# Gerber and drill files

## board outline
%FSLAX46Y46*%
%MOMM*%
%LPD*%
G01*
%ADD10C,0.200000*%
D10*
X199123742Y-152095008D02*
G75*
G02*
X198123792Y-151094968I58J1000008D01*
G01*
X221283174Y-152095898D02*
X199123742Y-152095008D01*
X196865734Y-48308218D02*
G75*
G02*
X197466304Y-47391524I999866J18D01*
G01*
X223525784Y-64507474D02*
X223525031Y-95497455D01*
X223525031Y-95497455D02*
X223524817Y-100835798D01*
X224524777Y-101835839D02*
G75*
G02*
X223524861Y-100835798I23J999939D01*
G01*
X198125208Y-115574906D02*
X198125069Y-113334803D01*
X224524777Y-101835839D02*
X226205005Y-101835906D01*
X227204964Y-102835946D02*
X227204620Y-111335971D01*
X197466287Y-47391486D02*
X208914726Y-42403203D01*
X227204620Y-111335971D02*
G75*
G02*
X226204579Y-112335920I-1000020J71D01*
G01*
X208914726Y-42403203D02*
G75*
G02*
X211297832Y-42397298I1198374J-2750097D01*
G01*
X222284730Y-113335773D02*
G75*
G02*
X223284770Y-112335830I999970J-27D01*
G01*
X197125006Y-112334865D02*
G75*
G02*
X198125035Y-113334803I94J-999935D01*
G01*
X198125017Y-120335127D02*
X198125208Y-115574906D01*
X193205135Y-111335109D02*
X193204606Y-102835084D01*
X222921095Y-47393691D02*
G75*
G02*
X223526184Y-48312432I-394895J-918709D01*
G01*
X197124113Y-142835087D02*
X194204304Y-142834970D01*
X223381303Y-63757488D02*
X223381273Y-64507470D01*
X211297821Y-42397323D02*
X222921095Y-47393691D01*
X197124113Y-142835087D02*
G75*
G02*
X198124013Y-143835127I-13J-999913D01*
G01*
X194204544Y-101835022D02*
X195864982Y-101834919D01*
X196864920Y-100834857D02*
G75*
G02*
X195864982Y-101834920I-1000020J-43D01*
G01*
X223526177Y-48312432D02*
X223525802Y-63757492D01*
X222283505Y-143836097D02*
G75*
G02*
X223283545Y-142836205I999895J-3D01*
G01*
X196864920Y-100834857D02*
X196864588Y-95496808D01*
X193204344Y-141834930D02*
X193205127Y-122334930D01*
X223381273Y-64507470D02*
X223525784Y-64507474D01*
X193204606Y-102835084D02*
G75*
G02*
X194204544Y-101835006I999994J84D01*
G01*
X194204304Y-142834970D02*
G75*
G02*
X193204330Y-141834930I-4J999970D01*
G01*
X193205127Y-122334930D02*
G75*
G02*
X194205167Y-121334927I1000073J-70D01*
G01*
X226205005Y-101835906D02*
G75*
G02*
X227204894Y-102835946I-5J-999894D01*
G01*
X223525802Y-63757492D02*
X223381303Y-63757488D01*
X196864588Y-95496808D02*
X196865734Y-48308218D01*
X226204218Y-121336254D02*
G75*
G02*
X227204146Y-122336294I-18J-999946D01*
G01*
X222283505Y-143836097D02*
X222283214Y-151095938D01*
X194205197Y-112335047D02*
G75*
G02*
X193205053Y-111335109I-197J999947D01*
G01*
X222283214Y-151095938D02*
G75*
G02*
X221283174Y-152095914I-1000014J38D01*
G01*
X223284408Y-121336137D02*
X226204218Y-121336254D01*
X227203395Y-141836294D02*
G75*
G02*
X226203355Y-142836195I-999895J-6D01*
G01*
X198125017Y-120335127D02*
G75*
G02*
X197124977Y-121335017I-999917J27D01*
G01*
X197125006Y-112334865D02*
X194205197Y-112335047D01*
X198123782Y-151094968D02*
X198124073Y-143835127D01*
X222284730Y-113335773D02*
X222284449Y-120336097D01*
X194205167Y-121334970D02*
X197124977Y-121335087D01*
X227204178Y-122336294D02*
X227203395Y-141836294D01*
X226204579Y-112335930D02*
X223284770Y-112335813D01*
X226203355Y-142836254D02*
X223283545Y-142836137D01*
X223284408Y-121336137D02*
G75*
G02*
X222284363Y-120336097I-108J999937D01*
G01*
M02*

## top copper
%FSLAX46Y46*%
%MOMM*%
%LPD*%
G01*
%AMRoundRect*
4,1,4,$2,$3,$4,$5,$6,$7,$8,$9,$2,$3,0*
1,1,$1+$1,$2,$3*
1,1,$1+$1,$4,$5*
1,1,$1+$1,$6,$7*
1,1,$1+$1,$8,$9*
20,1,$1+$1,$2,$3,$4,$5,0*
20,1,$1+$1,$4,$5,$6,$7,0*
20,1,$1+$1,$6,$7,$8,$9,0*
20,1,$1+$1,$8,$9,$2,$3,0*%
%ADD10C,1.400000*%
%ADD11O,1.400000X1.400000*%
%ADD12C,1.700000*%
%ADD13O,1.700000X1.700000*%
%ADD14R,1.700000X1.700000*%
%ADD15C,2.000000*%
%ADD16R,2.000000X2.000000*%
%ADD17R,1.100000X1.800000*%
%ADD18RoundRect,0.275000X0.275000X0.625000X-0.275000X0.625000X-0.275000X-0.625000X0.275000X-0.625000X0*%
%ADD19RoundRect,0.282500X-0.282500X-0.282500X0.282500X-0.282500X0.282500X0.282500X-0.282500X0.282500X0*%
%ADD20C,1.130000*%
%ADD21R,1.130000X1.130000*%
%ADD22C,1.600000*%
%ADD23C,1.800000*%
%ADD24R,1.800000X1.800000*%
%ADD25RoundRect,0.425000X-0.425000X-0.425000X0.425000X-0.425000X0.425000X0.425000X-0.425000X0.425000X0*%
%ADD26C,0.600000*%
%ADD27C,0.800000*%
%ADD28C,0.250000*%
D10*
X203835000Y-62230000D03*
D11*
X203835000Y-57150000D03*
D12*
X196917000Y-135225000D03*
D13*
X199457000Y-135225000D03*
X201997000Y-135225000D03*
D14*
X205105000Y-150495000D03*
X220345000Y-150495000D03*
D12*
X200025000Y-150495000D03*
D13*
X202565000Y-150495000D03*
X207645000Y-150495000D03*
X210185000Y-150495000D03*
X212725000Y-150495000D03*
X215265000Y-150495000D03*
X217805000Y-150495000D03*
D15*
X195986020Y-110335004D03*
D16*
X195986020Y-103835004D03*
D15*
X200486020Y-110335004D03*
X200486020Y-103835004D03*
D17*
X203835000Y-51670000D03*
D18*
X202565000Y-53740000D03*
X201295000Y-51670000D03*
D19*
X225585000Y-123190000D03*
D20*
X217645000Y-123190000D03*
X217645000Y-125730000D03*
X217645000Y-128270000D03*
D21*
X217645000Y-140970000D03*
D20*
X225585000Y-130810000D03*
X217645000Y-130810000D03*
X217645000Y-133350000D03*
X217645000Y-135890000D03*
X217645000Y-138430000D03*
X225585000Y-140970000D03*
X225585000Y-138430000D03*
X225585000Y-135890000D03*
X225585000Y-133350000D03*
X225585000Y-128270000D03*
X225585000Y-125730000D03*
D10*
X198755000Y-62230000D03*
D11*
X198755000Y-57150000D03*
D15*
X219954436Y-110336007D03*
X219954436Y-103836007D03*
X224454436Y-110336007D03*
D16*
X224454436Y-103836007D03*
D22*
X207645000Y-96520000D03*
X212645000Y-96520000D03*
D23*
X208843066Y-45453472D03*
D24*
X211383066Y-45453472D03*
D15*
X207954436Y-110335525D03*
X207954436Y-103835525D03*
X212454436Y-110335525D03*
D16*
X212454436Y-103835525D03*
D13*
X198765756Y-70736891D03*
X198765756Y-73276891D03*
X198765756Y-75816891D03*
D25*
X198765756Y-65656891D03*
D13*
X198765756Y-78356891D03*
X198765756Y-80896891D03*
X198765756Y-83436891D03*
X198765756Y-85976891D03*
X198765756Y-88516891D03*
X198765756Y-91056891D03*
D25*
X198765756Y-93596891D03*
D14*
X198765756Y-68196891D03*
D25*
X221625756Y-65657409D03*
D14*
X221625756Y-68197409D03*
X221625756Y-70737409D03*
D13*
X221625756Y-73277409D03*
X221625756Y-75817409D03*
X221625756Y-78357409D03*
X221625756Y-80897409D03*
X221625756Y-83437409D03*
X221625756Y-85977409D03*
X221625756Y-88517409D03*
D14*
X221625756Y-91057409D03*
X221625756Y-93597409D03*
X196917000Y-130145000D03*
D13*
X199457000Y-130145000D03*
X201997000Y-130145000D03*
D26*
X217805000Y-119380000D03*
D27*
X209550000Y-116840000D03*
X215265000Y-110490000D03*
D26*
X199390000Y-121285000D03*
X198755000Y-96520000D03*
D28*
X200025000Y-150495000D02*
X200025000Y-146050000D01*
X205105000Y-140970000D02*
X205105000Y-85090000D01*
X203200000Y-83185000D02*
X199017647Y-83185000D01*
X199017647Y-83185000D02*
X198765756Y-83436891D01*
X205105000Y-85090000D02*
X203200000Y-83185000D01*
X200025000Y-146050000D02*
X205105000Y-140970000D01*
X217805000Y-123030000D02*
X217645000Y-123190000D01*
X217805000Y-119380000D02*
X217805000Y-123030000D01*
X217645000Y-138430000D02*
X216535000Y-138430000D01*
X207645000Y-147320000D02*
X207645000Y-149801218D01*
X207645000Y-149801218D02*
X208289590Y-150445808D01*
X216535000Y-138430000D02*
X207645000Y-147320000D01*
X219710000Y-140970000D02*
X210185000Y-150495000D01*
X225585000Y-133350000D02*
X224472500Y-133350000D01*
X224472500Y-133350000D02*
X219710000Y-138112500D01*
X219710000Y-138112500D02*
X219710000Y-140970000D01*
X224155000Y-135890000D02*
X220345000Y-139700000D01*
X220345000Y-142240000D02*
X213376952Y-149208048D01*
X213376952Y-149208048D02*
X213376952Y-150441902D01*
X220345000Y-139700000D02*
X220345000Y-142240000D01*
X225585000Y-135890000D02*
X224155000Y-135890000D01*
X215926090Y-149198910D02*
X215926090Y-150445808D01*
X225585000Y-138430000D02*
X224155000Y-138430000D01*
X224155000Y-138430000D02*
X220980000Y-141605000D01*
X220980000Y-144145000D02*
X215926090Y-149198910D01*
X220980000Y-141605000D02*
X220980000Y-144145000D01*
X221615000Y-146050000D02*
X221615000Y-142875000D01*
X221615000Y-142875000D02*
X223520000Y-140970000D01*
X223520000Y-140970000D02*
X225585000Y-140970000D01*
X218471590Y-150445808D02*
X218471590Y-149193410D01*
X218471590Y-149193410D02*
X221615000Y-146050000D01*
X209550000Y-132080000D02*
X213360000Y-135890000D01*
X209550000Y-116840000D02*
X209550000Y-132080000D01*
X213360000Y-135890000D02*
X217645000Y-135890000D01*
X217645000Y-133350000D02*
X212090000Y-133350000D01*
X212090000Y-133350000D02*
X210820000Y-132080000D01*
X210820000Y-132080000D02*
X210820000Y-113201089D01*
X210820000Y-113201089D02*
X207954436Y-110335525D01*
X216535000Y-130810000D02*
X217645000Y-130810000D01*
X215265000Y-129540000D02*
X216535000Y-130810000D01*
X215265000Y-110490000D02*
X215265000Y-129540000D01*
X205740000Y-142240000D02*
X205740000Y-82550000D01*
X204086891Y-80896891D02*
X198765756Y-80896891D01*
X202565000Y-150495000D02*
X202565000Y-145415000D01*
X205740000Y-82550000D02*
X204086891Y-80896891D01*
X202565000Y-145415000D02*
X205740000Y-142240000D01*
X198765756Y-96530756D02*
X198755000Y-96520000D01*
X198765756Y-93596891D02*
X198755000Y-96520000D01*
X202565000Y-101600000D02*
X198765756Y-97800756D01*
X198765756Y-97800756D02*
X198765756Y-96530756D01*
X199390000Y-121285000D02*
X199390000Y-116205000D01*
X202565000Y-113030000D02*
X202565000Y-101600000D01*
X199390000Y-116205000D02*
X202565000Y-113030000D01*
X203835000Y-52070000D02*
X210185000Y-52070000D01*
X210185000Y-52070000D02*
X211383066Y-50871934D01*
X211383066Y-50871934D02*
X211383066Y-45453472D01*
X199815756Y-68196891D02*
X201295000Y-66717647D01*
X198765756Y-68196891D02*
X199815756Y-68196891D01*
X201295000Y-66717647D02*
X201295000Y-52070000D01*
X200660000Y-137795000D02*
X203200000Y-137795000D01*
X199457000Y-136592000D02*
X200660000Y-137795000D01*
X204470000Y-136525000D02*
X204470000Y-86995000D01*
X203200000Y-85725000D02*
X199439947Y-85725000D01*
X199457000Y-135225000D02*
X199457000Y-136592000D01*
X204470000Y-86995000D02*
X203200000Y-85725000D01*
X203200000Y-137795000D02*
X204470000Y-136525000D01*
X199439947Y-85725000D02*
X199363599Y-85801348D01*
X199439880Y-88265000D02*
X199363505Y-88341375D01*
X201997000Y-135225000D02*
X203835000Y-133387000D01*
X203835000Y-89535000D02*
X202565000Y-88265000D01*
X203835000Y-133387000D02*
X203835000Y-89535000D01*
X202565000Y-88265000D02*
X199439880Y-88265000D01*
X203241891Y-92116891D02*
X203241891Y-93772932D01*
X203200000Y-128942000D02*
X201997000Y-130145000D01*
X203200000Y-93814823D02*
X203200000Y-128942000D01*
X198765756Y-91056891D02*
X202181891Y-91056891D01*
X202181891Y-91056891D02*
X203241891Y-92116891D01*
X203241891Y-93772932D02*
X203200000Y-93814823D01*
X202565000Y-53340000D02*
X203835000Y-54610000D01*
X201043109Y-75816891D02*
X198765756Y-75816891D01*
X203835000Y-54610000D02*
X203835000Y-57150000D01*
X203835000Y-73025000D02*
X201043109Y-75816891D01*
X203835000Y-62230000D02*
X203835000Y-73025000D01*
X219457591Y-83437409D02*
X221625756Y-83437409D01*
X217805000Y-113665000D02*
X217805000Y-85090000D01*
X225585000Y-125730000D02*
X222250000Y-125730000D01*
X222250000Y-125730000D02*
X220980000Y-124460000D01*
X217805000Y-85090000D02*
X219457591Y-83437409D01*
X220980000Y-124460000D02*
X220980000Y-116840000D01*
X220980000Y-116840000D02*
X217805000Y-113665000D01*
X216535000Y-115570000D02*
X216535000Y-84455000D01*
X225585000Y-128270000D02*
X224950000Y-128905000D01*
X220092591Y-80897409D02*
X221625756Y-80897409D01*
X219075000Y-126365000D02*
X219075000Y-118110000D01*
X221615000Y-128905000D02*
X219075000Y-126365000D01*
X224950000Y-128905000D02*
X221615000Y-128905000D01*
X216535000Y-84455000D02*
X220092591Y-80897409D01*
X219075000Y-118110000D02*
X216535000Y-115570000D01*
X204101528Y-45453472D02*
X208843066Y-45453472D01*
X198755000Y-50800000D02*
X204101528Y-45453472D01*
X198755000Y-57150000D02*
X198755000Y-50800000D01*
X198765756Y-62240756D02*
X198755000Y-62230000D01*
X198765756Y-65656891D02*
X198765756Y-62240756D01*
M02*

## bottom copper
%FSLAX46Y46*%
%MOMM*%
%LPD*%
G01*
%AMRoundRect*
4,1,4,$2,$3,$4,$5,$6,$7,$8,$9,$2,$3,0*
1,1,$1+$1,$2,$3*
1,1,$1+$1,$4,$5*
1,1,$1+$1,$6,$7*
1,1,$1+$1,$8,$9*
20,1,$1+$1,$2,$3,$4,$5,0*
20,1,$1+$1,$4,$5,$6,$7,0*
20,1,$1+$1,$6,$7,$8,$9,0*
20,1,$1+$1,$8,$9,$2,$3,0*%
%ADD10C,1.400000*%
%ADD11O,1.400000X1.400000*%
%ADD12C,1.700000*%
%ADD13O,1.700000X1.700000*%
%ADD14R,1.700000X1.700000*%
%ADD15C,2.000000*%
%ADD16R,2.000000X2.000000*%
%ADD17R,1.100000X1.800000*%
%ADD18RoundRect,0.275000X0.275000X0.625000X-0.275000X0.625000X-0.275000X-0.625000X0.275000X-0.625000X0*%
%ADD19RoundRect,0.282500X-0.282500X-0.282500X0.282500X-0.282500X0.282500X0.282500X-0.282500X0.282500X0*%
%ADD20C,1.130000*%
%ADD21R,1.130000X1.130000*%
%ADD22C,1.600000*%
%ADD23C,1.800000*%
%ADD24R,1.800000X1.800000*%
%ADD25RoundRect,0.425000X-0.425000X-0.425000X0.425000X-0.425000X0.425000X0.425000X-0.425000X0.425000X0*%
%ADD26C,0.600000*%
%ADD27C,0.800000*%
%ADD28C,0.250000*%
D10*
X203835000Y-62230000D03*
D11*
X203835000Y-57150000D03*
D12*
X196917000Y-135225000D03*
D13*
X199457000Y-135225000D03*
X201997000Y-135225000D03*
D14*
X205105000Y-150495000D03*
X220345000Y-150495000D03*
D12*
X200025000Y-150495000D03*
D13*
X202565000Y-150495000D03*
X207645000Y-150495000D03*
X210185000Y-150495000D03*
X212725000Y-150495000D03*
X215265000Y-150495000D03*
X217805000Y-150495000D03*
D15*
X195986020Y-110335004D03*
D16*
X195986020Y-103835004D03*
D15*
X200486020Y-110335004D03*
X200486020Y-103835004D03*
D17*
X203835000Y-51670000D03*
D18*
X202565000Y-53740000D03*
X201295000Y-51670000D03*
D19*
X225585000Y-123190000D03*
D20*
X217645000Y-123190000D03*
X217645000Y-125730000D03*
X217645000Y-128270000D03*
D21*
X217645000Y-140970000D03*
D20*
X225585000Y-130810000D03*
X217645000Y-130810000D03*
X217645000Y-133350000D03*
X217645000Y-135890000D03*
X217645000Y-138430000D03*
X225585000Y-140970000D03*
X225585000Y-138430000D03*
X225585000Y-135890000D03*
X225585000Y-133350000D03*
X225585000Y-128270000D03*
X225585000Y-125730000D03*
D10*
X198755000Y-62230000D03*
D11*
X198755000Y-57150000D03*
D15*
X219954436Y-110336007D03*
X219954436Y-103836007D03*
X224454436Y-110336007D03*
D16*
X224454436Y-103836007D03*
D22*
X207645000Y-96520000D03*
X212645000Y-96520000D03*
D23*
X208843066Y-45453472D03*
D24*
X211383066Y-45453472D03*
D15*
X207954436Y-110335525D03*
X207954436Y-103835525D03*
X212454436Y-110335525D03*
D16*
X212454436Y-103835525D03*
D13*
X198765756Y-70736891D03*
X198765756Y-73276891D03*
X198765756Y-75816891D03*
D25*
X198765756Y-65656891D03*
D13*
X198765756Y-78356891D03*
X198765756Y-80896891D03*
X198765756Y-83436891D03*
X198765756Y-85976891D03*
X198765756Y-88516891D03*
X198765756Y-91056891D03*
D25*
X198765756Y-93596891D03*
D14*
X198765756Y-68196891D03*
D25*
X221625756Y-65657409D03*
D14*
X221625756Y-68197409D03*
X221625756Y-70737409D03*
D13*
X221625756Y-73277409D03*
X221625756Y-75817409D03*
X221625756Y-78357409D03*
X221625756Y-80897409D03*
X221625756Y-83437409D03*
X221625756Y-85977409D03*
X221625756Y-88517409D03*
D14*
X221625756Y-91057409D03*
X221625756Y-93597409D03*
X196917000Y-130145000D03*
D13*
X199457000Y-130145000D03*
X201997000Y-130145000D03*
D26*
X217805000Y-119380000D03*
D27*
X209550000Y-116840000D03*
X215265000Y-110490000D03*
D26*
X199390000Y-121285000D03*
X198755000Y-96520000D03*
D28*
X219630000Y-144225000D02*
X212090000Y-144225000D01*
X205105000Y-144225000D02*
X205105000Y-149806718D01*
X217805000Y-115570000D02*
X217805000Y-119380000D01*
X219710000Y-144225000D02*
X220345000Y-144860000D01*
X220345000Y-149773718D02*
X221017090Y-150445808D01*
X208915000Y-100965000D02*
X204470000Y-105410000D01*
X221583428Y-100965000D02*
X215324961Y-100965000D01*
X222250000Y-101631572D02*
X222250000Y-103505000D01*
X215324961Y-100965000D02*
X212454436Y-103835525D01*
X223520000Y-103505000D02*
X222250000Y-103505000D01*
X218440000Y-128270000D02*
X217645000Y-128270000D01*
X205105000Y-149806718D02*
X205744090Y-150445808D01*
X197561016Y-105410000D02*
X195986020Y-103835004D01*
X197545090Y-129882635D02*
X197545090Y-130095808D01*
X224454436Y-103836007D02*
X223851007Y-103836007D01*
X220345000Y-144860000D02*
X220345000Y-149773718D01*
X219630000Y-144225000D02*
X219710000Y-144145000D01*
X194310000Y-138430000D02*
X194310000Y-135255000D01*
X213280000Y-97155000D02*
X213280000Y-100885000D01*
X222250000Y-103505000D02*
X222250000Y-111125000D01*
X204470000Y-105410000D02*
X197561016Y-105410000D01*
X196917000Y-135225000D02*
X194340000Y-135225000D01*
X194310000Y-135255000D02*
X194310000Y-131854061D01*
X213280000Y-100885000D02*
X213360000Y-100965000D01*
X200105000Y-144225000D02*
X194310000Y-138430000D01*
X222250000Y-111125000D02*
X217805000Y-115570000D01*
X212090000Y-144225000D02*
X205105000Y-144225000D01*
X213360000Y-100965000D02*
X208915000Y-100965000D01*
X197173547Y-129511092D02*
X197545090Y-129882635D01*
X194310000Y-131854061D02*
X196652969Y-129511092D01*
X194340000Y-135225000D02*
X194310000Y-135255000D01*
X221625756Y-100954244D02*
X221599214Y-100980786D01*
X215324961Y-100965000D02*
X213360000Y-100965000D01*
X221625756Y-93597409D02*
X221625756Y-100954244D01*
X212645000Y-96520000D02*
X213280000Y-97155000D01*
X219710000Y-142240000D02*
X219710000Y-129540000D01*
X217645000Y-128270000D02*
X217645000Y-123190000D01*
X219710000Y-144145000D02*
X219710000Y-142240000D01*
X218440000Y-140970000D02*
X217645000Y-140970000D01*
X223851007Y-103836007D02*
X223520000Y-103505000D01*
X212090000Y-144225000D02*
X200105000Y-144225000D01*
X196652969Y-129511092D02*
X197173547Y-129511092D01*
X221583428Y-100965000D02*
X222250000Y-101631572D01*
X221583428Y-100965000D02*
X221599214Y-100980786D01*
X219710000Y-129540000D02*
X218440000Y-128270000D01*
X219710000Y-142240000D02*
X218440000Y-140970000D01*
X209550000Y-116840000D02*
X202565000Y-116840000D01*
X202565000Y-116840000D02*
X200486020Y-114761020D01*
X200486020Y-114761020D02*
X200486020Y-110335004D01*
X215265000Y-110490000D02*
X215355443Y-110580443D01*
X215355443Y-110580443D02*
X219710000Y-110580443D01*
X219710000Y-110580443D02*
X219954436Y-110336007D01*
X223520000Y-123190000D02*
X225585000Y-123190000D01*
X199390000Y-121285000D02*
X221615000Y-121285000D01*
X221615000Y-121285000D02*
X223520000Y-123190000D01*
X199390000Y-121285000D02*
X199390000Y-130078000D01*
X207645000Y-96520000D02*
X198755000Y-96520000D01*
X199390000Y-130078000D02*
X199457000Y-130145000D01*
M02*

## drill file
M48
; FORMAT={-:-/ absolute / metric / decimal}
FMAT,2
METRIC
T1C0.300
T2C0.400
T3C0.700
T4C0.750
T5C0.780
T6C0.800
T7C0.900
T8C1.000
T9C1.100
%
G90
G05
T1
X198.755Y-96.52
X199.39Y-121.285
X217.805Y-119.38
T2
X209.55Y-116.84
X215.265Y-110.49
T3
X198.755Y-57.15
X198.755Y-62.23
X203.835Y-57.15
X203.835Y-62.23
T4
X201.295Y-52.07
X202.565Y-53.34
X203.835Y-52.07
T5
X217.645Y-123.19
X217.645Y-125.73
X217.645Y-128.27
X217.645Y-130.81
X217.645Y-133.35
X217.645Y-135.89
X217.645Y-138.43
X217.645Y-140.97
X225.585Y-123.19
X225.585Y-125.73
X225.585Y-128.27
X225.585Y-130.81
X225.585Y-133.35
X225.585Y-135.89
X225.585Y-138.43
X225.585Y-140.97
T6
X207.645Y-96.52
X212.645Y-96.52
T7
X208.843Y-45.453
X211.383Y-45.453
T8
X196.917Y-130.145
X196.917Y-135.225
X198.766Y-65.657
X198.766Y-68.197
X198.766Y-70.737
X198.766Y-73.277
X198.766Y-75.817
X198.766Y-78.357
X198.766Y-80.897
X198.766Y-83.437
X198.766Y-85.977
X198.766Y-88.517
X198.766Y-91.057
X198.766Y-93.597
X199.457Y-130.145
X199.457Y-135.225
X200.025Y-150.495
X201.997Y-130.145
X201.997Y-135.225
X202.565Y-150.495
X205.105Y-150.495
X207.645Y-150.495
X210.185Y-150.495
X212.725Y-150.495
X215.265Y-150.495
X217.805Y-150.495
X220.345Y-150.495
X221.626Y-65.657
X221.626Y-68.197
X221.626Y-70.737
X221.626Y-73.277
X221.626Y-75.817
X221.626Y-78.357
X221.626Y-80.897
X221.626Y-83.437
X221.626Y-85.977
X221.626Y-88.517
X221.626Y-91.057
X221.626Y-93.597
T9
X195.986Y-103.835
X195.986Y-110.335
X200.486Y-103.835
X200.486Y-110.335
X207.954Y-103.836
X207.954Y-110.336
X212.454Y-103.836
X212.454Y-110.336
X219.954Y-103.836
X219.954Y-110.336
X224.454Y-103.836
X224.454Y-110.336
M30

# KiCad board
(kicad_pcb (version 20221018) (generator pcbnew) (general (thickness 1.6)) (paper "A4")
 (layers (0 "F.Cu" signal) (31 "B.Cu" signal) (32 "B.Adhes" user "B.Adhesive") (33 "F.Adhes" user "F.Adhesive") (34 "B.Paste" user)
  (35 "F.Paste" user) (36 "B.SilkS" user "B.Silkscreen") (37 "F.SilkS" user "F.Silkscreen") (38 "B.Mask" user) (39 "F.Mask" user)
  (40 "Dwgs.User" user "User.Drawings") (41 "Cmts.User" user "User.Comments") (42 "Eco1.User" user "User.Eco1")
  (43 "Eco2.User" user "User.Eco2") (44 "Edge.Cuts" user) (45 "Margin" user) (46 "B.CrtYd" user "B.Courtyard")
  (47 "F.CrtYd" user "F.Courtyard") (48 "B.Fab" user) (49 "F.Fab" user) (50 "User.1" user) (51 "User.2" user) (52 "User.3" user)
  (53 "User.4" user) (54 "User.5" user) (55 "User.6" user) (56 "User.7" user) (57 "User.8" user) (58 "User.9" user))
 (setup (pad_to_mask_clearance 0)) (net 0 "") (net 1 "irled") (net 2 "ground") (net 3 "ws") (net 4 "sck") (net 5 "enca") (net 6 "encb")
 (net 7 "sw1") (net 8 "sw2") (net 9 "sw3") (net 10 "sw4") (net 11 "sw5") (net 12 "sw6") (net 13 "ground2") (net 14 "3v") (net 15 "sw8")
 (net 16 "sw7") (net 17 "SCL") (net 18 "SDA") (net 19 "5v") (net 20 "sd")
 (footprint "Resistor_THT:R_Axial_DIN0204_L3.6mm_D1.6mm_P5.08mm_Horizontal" (layer "F.Cu") (at 203.835 62.23 90)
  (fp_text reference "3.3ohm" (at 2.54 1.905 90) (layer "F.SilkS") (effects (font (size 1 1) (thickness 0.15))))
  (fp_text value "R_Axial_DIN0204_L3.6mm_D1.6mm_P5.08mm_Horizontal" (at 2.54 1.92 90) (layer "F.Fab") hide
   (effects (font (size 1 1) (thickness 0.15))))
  (pad "1" thru_hole circle (at 0 0 90) (size 1.4 1.4) (drill 0.7) (layers "*.Cu" "*.Mask") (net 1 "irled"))
  (pad "2" thru_hole oval (at 5.08 0 90) (size 1.4 1.4) (drill 0.7) (layers "*.Cu" "*.Mask") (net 1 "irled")))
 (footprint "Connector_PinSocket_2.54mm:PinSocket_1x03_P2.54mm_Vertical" (layer "F.Cu") (at 196.917 135.225 90)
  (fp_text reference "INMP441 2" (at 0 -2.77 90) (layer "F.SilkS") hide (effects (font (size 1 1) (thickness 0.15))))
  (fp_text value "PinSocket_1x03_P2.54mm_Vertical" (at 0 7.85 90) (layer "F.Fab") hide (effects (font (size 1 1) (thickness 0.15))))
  (pad "1" thru_hole circle (at 0 0 90) (size 1.7 1.7) (drill 1) (layers "*.Cu" "*.Mask") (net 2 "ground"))
  (pad "2" thru_hole oval (at 0 2.54 90) (size 1.7 1.7) (drill 1) (layers "*.Cu" "*.Mask") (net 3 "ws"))
  (pad "3" thru_hole oval (at 0 5.08 90) (size 1.7 1.7) (drill 1) (layers "*.Cu" "*.Mask") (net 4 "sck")))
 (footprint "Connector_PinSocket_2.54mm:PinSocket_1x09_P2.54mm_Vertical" (layer "F.Cu") (at 200.025 150.495 90)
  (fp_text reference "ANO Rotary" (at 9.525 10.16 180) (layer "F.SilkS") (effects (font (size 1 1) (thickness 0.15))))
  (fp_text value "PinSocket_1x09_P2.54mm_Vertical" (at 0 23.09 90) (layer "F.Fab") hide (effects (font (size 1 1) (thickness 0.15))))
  (pad "COMA" thru_hole rect (at 0 5.08 90) (size 1.7 1.7) (drill 1) (layers "*.Cu" "*.Mask") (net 2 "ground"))
  (pad "COMB" thru_hole rect (at 0 20.32 90) (size 1.7 1.7) (drill 1) (layers "*.Cu" "*.Mask") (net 2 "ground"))
  (pad "ENCA" thru_hole circle (at 0 0 90) (size 1.7 1.7) (drill 1) (layers "*.Cu" "*.Mask") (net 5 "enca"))
  (pad "ENCB" thru_hole oval (at 0 2.54 90) (size 1.7 1.7) (drill 1) (layers "*.Cu" "*.Mask") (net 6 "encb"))
  (pad "SW1" thru_hole oval (at 0 7.62 90) (size 1.7 1.7) (drill 1) (layers "*.Cu" "*.Mask") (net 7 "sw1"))
  (pad "SW2" thru_hole oval (at 0 10.16 90) (size 1.7 1.7) (drill 1) (layers "*.Cu" "*.Mask") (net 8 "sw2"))
  (pad "SW3" thru_hole oval (at 0 12.7 90) (size 1.7 1.7) (drill 1) (layers "*.Cu" "*.Mask") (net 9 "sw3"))
  (pad "SW4" thru_hole oval (at 0 15.24 90) (size 1.7 1.7) (drill 1) (layers "*.Cu" "*.Mask") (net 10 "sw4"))
  (pad "SW5" thru_hole oval (at 0 17.78 90) (size 1.7 1.7) (drill 1) (layers "*.Cu" "*.Mask") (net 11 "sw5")))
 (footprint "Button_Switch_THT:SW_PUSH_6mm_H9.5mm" (layer "F.Cu") (at 195.98602 110.335004 90)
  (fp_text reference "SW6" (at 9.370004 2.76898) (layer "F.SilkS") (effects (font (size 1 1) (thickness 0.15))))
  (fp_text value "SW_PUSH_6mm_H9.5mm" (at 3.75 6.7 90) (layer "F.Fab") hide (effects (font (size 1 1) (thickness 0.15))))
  (pad "1" thru_hole circle (at 0 0 180) (size 2 2) (drill 1.1) (layers "*.Cu" "*.Mask"))
  (pad "1" thru_hole rect (at 6.5 0 180) (size 2 2) (drill 1.1) (layers "*.Cu" "*.Mask") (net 2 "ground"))
  (pad "2" thru_hole circle (at 0 4.5 180) (size 2 2) (drill 1.1) (layers "*.Cu" "*.Mask") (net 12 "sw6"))
  (pad "2" thru_hole circle (at 6.5 4.5 180) (size 2 2) (drill 1.1) (layers "*.Cu" "*.Mask")))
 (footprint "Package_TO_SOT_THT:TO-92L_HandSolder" (layer "F.Cu") (at 203.835 52.07 180)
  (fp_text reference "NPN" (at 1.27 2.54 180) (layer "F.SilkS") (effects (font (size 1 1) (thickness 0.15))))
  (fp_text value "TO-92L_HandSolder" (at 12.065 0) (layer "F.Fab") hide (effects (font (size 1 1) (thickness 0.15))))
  (pad "1" thru_hole rect (at 0 0 180) (size 1.1 1.8) (drill 0.75 (offset 0 0.4)) (layers "*.Cu" "*.Mask") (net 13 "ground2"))
  (pad "2" thru_hole roundrect (at 1.27 -1.27 180) (size 1.1 1.8) (drill 0.75 (offset 0 -0.4)) (layers "*.Cu" "*.Mask")
   (roundrect_rratio 0.25) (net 1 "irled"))
  (pad "3" thru_hole roundrect (at 2.54 0 180) (size 1.1 1.8) (drill 0.75 (offset 0 0.4)) (layers "*.Cu" "*.Mask") (roundrect_rratio 0.25)
   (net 13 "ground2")))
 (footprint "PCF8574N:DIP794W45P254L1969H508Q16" (layer "F.Cu") (at 221.615 132.08)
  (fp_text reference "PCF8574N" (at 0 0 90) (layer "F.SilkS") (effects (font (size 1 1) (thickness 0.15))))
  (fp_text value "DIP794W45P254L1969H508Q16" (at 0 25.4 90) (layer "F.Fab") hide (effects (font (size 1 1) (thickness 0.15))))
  (pad "16" thru_hole roundrect (at 3.97 -8.89) (size 1.13 1.13) (drill 0.78) (layers "*.Cu" "*.Mask") (roundrect_rratio 0.25) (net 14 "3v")
   (solder_mask_margin 0.102))
  (pad "A0" thru_hole circle (at -3.97 -8.89) (size 1.13 1.13) (drill 0.78) (layers "*.Cu" "*.Mask") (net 2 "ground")
   (solder_mask_margin 0.102))
  (pad "A1" thru_hole circle (at -3.97 -6.35) (size 1.13 1.13) (drill 0.78) (layers "*.Cu" "*.Mask") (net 2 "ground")
   (solder_mask_margin 0.102))
  (pad "A2" thru_hole circle (at -3.97 -3.81) (size 1.13 1.13) (drill 0.78) (layers "*.Cu" "*.Mask") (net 2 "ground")
   (solder_mask_margin 0.102))
  (pad "GND" thru_hole rect (at -3.97 8.89) (size 1.13 1.13) (drill 0.78) (layers "*.Cu" "*.Mask") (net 2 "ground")
   (solder_mask_margin 0.102))
  (pad "INT" thru_hole circle (at 3.97 -1.27) (size 1.13 1.13) (drill 0.78) (layers "*.Cu" "*.Mask") (solder_mask_margin 0.102))
  (pad "P0" thru_hole circle (at -3.97 -1.27) (size 1.13 1.13) (drill 0.78) (layers "*.Cu" "*.Mask") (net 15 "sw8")
   (solder_mask_margin 0.102))
  (pad "P1" thru_hole circle (at -3.97 1.27) (size 1.13 1.13) (drill 0.78) (layers "*.Cu" "*.Mask") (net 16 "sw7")
   (solder_mask_margin 0.102))
  (pad "P2" thru_hole circle (at -3.97 3.81) (size 1.13 1.13) (drill 0.78) (layers "*.Cu" "*.Mask") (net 12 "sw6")
   (solder_mask_margin 0.102))
  (pad "P3" thru_hole circle (at -3.97 6.35) (size 1.13 1.13) (drill 0.78) (layers "*.Cu" "*.Mask") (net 7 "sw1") (solder_mask_margin 0.102))
  (pad "P4" thru_hole circle (at 3.97 8.89) (size 1.13 1.13) (drill 0.78) (layers "*.Cu" "*.Mask") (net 11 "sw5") (solder_mask_margin 0.102))
  (pad "P5" thru_hole circle (at 3.97 6.35) (size 1.13 1.13) (drill 0.78) (layers "*.Cu" "*.Mask") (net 10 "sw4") (solder_mask_margin 0.102))
  (pad "P6" thru_hole circle (at 3.97 3.81) (size 1.13 1.13) (drill 0.78) (layers "*.Cu" "*.Mask") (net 9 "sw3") (solder_mask_margin 0.102))
  (pad "P7" thru_hole circle (at 3.97 1.27) (size 1.13 1.13) (drill 0.78) (layers "*.Cu" "*.Mask") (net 8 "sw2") (solder_mask_margin 0.102))
  (pad "SCL" thru_hole circle (at 3.97 -3.81) (size 1.13 1.13) (drill 0.78) (layers "*.Cu" "*.Mask") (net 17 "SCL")
   (solder_mask_margin 0.102))
  (pad "SDA" thru_hole circle (at 3.97 -6.35) (size 1.13 1.13) (drill 0.78) (layers "*.Cu" "*.Mask") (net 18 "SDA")
   (solder_mask_margin 0.102)))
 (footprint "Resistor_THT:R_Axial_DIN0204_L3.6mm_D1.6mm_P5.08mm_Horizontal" (layer "F.Cu") (at 198.755 62.23 90)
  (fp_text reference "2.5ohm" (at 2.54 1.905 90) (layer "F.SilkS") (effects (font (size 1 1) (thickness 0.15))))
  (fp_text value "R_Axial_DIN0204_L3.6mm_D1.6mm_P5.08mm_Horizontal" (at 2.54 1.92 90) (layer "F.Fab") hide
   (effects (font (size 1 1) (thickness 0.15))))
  (pad "1" thru_hole circle (at 0 0 90) (size 1.4 1.4) (drill 0.7) (layers "*.Cu" "*.Mask") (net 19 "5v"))
  (pad "2" thru_hole oval (at 5.08 0 90) (size 1.4 1.4) (drill 0.7) (layers "*.Cu" "*.Mask") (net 19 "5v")))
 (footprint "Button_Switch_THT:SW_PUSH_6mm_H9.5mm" (layer "F.Cu") (at 219.954436 110.336007 90)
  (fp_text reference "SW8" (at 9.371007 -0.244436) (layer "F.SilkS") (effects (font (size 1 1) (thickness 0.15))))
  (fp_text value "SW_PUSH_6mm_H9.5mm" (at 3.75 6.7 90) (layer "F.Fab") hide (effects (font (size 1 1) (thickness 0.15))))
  (pad "1" thru_hole circle (at 0 0 180) (size 2 2) (drill 1.1) (layers "*.Cu" "*.Mask") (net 15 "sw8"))
  (pad "1" thru_hole circle (at 6.5 0 180) (size 2 2) (drill 1.1) (layers "*.Cu" "*.Mask"))
  (pad "2" thru_hole circle (at 0 4.5 180) (size 2 2) (drill 1.1) (layers "*.Cu" "*.Mask"))
  (pad "2" thru_hole rect (at 6.5 4.5 180) (size 2 2) (drill 1.1) (layers "*.Cu" "*.Mask") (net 2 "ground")))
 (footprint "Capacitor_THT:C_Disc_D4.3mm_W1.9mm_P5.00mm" (layer "F.Cu") (at 207.645 96.52)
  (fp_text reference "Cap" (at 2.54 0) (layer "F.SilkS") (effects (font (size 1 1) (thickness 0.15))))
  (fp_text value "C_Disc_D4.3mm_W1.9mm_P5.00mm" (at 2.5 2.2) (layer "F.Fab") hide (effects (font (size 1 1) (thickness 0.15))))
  (pad "1" thru_hole circle (at 0 0) (size 1.6 1.6) (drill 0.8) (layers "*.Cu" "*.Mask") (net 14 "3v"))
  (pad "2" thru_hole circle (at 5 0) (size 1.6 1.6) (drill 0.8) (layers "*.Cu" "*.Mask") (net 2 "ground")))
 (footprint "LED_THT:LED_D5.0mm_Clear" (layer "F.Cu") (at 208.843066 45.453472)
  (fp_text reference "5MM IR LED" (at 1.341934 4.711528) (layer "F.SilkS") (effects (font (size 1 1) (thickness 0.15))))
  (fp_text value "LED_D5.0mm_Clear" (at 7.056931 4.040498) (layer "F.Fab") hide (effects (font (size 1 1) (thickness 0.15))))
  (pad "1" thru_hole circle (at 0 0) (size 1.8 1.8) (drill 0.9) (layers "*.Cu" "*.Mask") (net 19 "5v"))
  (pad "2" thru_hole rect (at 2.54 0) (size 1.8 1.8) (drill 0.9) (layers "*.Cu" "*.Mask") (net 13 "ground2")))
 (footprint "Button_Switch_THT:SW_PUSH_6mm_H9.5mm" (layer "F.Cu") (at 207.954436 110.335525 90)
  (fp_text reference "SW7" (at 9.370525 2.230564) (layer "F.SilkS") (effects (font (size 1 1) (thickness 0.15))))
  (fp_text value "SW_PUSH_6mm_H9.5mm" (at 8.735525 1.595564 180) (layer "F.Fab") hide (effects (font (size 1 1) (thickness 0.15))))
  (pad "1" thru_hole circle (at 0 0 180) (size 2 2) (drill 1.1) (layers "*.Cu" "*.Mask") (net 16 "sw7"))
  (pad "1" thru_hole circle (at 6.5 0 180) (size 2 2) (drill 1.1) (layers "*.Cu" "*.Mask"))
  (pad "2" thru_hole circle (at 0 4.5 180) (size 2 2) (drill 1.1) (layers "*.Cu" "*.Mask"))
  (pad "2" thru_hole rect (at 6.5 4.5 180) (size 2 2) (drill 1.1) (layers "*.Cu" "*.Mask") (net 2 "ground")))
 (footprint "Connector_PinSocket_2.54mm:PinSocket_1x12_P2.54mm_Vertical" (layer "F.Cu") (at 198.765756 65.656891)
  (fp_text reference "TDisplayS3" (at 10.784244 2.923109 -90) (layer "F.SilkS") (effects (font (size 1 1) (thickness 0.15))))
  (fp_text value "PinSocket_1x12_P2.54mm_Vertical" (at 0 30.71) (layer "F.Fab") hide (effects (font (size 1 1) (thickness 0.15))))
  (pad "3" thru_hole oval (at 0 5.08) (size 1.7 1.7) (drill 1) (layers "*.Cu" "*.Mask"))
  (pad "4" thru_hole oval (at 0 7.62) (size 1.7 1.7) (drill 1) (layers "*.Cu" "*.Mask"))
  (pad "5" thru_hole oval (at 0 10.16) (size 1.7 1.7) (drill 1) (layers "*.Cu" "*.Mask") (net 1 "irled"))
  (pad "5v" thru_hole roundrect (at 0 0) (size 1.7 1.7) (drill 1) (layers "*.Cu" "*.Mask") (roundrect_rratio 0.25) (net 19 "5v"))
  (pad "6" thru_hole oval (at 0 12.7) (size 1.7 1.7) (drill 1) (layers "*.Cu" "*.Mask"))
  (pad "7" thru_hole oval (at 0 15.24) (size 1.7 1.7) (drill 1) (layers "*.Cu" "*.Mask") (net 6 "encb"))
  (pad "8" thru_hole oval (at 0 17.78) (size 1.7 1.7) (drill 1) (layers "*.Cu" "*.Mask") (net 5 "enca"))
  (pad "9" thru_hole oval (at 0 20.32) (size 1.7 1.7) (drill 1) (layers "*.Cu" "*.Mask") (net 3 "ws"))
  (pad "10" thru_hole oval (at 0 22.86) (size 1.7 1.7) (drill 1) (layers "*.Cu" "*.Mask") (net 4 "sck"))
  (pad "11" thru_hole oval (at 0 25.4) (size 1.7 1.7) (drill 1) (layers "*.Cu" "*.Mask") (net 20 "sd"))
  (pad "12" thru_hole roundrect (at 0 27.94) (size 1.7 1.7) (drill 1) (layers "*.Cu" "*.Mask") (roundrect_rratio 0.25) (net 14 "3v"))
  (pad "gnd" thru_hole rect (at 0 2.54) (size 1.7 1.7) (drill 1) (layers "*.Cu" "*.Mask") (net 13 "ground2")))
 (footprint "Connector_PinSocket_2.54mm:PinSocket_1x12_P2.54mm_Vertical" (layer "F.Cu") (at 221.625756 65.657409)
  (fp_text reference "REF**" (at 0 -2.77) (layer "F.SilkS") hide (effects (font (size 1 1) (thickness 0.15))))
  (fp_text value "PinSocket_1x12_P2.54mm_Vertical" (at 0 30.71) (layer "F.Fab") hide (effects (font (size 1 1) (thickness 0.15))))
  (pad "1" thru_hole roundrect (at 0 0) (size 1.7 1.7) (drill 1) (layers "*.Cu" "*.Mask") (roundrect_rratio 0.25))
  (pad "2" thru_hole rect (at 0 2.54) (size 1.7 1.7) (drill 1) (layers "*.Cu" "*.Mask"))
  (pad "3" thru_hole rect (at 0 5.08) (size 1.7 1.7) (drill 1) (layers "*.Cu" "*.Mask"))
  (pad "4" thru_hole oval (at 0 7.62) (size 1.7 1.7) (drill 1) (layers "*.Cu" "*.Mask"))
  (pad "5" thru_hole oval (at 0 10.16) (size 1.7 1.7) (drill 1) (layers "*.Cu" "*.Mask"))
  (pad "6" thru_hole oval (at 0 12.7) (size 1.7 1.7) (drill 1) (layers "*.Cu" "*.Mask"))
  (pad "7" thru_hole oval (at 0 15.24) (size 1.7 1.7) (drill 1) (layers "*.Cu" "*.Mask") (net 17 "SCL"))
  (pad "8" thru_hole oval (at 0 17.78) (size 1.7 1.7) (drill 1) (layers "*.Cu" "*.Mask") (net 18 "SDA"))
  (pad "9" thru_hole oval (at 0 20.32) (size 1.7 1.7) (drill 1) (layers "*.Cu" "*.Mask"))
  (pad "10" thru_hole oval (at 0 22.86) (size 1.7 1.7) (drill 1) (layers "*.Cu" "*.Mask"))
  (pad "11" thru_hole rect (at 0 25.4) (size 1.7 1.7) (drill 1) (layers "*.Cu" "*.Mask"))
  (pad "12" thru_hole rect (at 0 27.94) (size 1.7 1.7) (drill 1) (layers "*.Cu" "*.Mask") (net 2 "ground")))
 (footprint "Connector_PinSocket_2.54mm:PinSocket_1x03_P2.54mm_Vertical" (layer "F.Cu") (at 196.917 130.145 90)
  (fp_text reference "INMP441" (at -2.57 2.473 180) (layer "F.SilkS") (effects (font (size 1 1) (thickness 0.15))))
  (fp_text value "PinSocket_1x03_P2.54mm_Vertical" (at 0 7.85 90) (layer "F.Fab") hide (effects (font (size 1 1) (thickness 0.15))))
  (pad "1" thru_hole rect (at 0 0 90) (size 1.7 1.7) (drill 1) (layers "*.Cu" "*.Mask") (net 2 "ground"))
  (pad "2" thru_hole oval (at 0 2.54 90) (size 1.7 1.7) (drill 1) (layers "*.Cu" "*.Mask") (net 14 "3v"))
  (pad "3" thru_hole oval (at 0 5.08 90) (size 1.7 1.7) (drill 1) (layers "*.Cu" "*.Mask") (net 20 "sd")))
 (gr_arc (start 199.123742 152.095008) (mid 198.416656 151.802081) (end 198.123782 151.094968) (stroke (width 0.2) (type solid))
  (layer "Edge.Cuts"))
 (gr_line (start 221.283174 152.095898) (end 199.123742 152.095008) (stroke (width 0.2) (type solid)) (layer "Edge.Cuts"))
 (gr_arc (start 196.865734 48.308218) (mid 197.029233 47.760245) (end 197.466287 47.391486) (stroke (width 0.2) (type solid))
  (layer "Edge.Cuts"))
 (gr_line (start 223.525784 64.507474) (end 223.525031 95.497455) (stroke (width 0.2) (type solid)) (layer "Edge.Cuts"))
 (gr_line (start 223.525031 95.497455) (end 223.524817 100.835798) (stroke (width 0.2) (type solid)) (layer "Edge.Cuts"))
 (gr_arc (start 224.524777 101.835839) (mid 223.817657 101.542926) (end 223.524817 100.835798) (stroke (width 0.2) (type solid))
  (layer "Edge.Cuts"))
 (gr_line (start 198.125208 115.574906) (end 198.125069 113.334803) (stroke (width 0.2) (type solid)) (layer "Edge.Cuts"))
 (gr_line (start 224.524777 101.835839) (end 226.205005 101.835906) (stroke (width 0.2) (type solid)) (layer "Edge.Cuts"))
 (gr_line (start 227.204964 102.835946) (end 227.20462 111.335971) (stroke (width 0.2) (type solid)) (layer "Edge.Cuts"))
 (gr_line (start 197.466287 47.391486) (end 208.914726 42.403203) (stroke (width 0.2) (type solid)) (layer "Edge.Cuts"))
 (gr_arc (start 227.20462 111.335971) (mid 226.911688 112.043053) (end 226.204579 112.33593) (stroke (width 0.2) (type solid))
  (layer "Edge.Cuts"))
 (gr_arc (start 208.914726 42.403203) (mid 210.105667 42.15347) (end 211.297821 42.397323) (stroke (width 0.2) (type solid))
  (layer "Edge.Cuts"))
 (gr_arc (start 222.28473 113.335773) (mid 222.577649 112.62868) (end 223.28477 112.335813) (stroke (width 0.2) (type solid))
  (layer "Edge.Cuts"))
 (gr_arc (start 197.125006 112.334865) (mid 197.832164 112.627701) (end 198.125069 113.334803) (stroke (width 0.2) (type solid))
  (layer "Edge.Cuts"))
 (gr_line (start 198.125017 120.335127) (end 198.125208 115.574906) (stroke (width 0.2) (type solid)) (layer "Edge.Cuts"))
 (gr_line (start 193.205135 111.335109) (end 193.204606 102.835084) (stroke (width 0.2) (type solid)) (layer "Edge.Cuts"))
 (gr_arc (start 222.921095 47.393691) (mid 223.361331 47.762377) (end 223.526177 48.312432) (stroke (width 0.2) (type solid))
  (layer "Edge.Cuts"))
 (gr_line (start 197.124113 142.835087) (end 194.204304 142.83497) (stroke (width 0.2) (type solid)) (layer "Edge.Cuts"))
 (gr_line (start 223.381303 63.757488) (end 223.381273 64.50747) (stroke (width 0.2) (type solid)) (layer "Edge.Cuts"))
 (gr_line (start 211.297821 42.397323) (end 222.921095 47.393691) (stroke (width 0.2) (type solid)) (layer "Edge.Cuts"))
 (gr_arc (start 197.124113 142.835087) (mid 197.83123 143.127998) (end 198.124073 143.835127) (stroke (width 0.2) (type solid))
  (layer "Edge.Cuts"))
 (gr_line (start 194.204544 101.835022) (end 195.864982 101.834919) (stroke (width 0.2) (type solid)) (layer "Edge.Cuts"))
 (gr_arc (start 196.86492 100.834857) (mid 196.572065 101.541977) (end 195.864982 101.834919) (stroke (width 0.2) (type solid))
  (layer "Edge.Cuts"))
 (gr_line (start 223.526177 48.312432) (end 223.525802 63.757492) (stroke (width 0.2) (type solid)) (layer "Edge.Cuts"))
 (gr_arc (start 222.283505 143.836097) (mid 222.576414 143.12898) (end 223.283545 142.836137) (stroke (width 0.2) (type solid))
  (layer "Edge.Cuts"))
 (gr_line (start 196.86492 100.834857) (end 196.864588 95.496808) (stroke (width 0.2) (type solid)) (layer "Edge.Cuts"))
 (gr_line (start 193.204344 141.83493) (end 193.205127 122.33493) (stroke (width 0.2) (type solid)) (layer "Edge.Cuts"))
 (gr_line (start 223.381273 64.50747) (end 223.525784 64.507474) (stroke (width 0.2) (type solid)) (layer "Edge.Cuts"))
 (gr_arc (start 193.204606 102.835084) (mid 193.497448 102.127947) (end 194.204544 101.835022) (stroke (width 0.2) (type solid))
  (layer "Edge.Cuts"))
 (gr_arc (start 194.204304 142.83497) (mid 193.497191 142.542062) (end 193.204344 141.83493) (stroke (width 0.2) (type solid))
  (layer "Edge.Cuts"))
 (gr_arc (start 193.205127 122.33493) (mid 193.498061 121.627864) (end 194.205167 121.33497) (stroke (width 0.2) (type solid))
  (layer "Edge.Cuts"))
 (gr_arc (start 226.205005 101.835906) (mid 226.912121 102.128815) (end 227.204964 102.835946) (stroke (width 0.2) (type solid))
  (layer "Edge.Cuts"))
 (gr_line (start 223.525802 63.757492) (end 223.381303 63.757488) (stroke (width 0.2) (type solid)) (layer "Edge.Cuts"))
 (gr_line (start 196.864588 95.496808) (end 196.865734 48.308218) (stroke (width 0.2) (type solid)) (layer "Edge.Cuts"))
 (gr_arc (start 226.204218 121.336254) (mid 226.911344 121.629165) (end 227.204178 122.336294) (stroke (width 0.2) (type solid))
  (layer "Edge.Cuts"))
 (gr_line (start 222.283505 143.836097) (end 222.283214 151.095938) (stroke (width 0.2) (type solid)) (layer "Edge.Cuts"))
 (gr_arc (start 194.205197 112.335047) (mid 193.498033 112.042213) (end 193.205135 111.335109) (stroke (width 0.2) (type solid))
  (layer "Edge.Cuts"))
 (gr_arc (start 222.283214 151.095938) (mid 221.990294 151.803039) (end 221.283174 152.095898) (stroke (width 0.2) (type solid))
  (layer "Edge.Cuts"))
 (gr_line (start 223.284408 121.336137) (end 226.204218 121.336254) (stroke (width 0.2) (type solid)) (layer "Edge.Cuts"))
 (gr_arc (start 227.203395 141.836294) (mid 226.910489 142.543417) (end 226.203355 142.836254) (stroke (width 0.2) (type solid))
  (layer "Edge.Cuts"))
 (gr_arc (start 198.125017 120.335127) (mid 197.832101 121.042236) (end 197.124977 121.335087) (stroke (width 0.2) (type solid))
  (layer "Edge.Cuts"))
 (gr_line (start 197.125006 112.334865) (end 194.205197 112.335047) (stroke (width 0.2) (type solid)) (layer "Edge.Cuts"))
 (gr_line (start 198.123782 151.094968) (end 198.124073 143.835127) (stroke (width 0.2) (type solid)) (layer "Edge.Cuts"))
 (gr_line (start 222.28473 113.335773) (end 222.284449 120.336097) (stroke (width 0.2) (type solid)) (layer "Edge.Cuts"))
 (gr_line (start 194.205167 121.33497) (end 197.124977 121.335087) (stroke (width 0.2) (type solid)) (layer "Edge.Cuts"))
 (gr_line (start 227.204178 122.336294) (end 227.203395 141.836294) (stroke (width 0.2) (type solid)) (layer "Edge.Cuts"))
 (gr_line (start 226.204579 112.33593) (end 223.28477 112.335813) (stroke (width 0.2) (type solid)) (layer "Edge.Cuts"))
 (gr_line (start 226.203355 142.836254) (end 223.283545 142.836137) (stroke (width 0.2) (type solid)) (layer "Edge.Cuts"))
 (gr_arc (start 223.284408 121.336137) (mid 222.577269 121.043235) (end 222.284449 120.336097) (stroke (width 0.2) (type solid))
  (layer "Edge.Cuts"))
 (segment (start 200.025 150.495) (end 200.025 146.05) (width 0.25) (layer "F.Cu") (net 5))
 (segment (start 205.105 140.97) (end 205.105 85.09) (width 0.25) (layer "F.Cu") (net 5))
 (segment (start 203.2 83.185) (end 199.017647 83.185) (width 0.25) (layer "F.Cu") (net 5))
 (segment (start 199.017647 83.185) (end 198.765756 83.436891) (width 0.25) (layer "F.Cu") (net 5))
 (segment (start 205.105 85.09) (end 203.2 83.185) (width 0.25) (layer "F.Cu") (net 5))
 (segment (start 200.025 146.05) (end 205.105 140.97) (width 0.25) (layer "F.Cu") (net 5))
 (segment (start 217.805 123.03) (end 217.645 123.19) (width 0.25) (layer "F.Cu") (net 2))
 (segment (start 217.805 119.38) (end 217.805 123.03) (width 0.25) (layer "F.Cu") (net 2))
 (via (at 217.805 119.38) (size 0.6) (drill 0.3) (layers "F.Cu" "B.Cu") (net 2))
 (segment (start 219.63 144.225) (end 212.09 144.225) (width 0.25) (layer "B.Cu") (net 2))
 (segment (start 205.105 144.225) (end 205.105 149.806718) (width 0.25) (layer "B.Cu") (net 2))
 (segment (start 217.805 115.57) (end 217.805 119.38) (width 0.25) (layer "B.Cu") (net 2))
 (segment (start 219.71 144.225) (end 220.345 144.86) (width 0.25) (layer "B.Cu") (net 2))
 (segment (start 220.345 149.773718) (end 221.01709 150.445808) (width 0.25) (layer "B.Cu") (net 2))
 (segment (start 208.915 100.965) (end 204.47 105.41) (width 0.25) (layer "B.Cu") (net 2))
 (segment (start 221.583428 100.965) (end 215.324961 100.965) (width 0.25) (layer "B.Cu") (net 2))
 (segment (start 222.25 101.631572) (end 222.25 103.505) (width 0.25) (layer "B.Cu") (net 2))
 (segment (start 215.324961 100.965) (end 212.454436 103.835525) (width 0.25) (layer "B.Cu") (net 2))
 (segment (start 223.52 103.505) (end 222.25 103.505) (width 0.25) (layer "B.Cu") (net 2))
 (segment (start 218.44 128.27) (end 217.645 128.27) (width 0.25) (layer "B.Cu") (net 2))
 (segment (start 205.105 149.806718) (end 205.74409 150.445808) (width 0.25) (layer "B.Cu") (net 2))
 (segment (start 197.561016 105.41) (end 195.98602 103.835004) (width 0.25) (layer "B.Cu") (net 2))
 (segment (start 197.54509 129.882635) (end 197.54509 130.095808) (width 0.25) (layer "B.Cu") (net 2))
 (segment (start 224.454436 103.836007) (end 223.851007 103.836007) (width 0.25) (layer "B.Cu") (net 2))
 (segment (start 220.345 144.86) (end 220.345 149.773718) (width 0.25) (layer "B.Cu") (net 2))
 (segment (start 219.63 144.225) (end 219.71 144.145) (width 0.25) (layer "B.Cu") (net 2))
 (segment (start 194.31 138.43) (end 194.31 135.255) (width 0.25) (layer "B.Cu") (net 2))
 (segment (start 213.28 97.155) (end 213.28 100.885) (width 0.25) (layer "B.Cu") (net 2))
 (segment (start 222.25 103.505) (end 222.25 111.125) (width 0.25) (layer "B.Cu") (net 2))
 (segment (start 204.47 105.41) (end 197.561016 105.41) (width 0.25) (layer "B.Cu") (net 2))
 (segment (start 196.917 135.225) (end 194.34 135.225) (width 0.25) (layer "B.Cu") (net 2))
 (segment (start 194.31 135.255) (end 194.31 131.854061) (width 0.25) (layer "B.Cu") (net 2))
 (segment (start 213.28 100.885) (end 213.36 100.965) (width 0.25) (layer "B.Cu") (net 2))
 (segment (start 200.105 144.225) (end 194.31 138.43) (width 0.25) (layer "B.Cu") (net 2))
 (segment (start 222.25 111.125) (end 217.805 115.57) (width 0.25) (layer "B.Cu") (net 2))
 (segment (start 212.09 144.225) (end 205.105 144.225) (width 0.25) (layer "B.Cu") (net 2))
 (segment (start 213.36 100.965) (end 208.915 100.965) (width 0.25) (layer "B.Cu") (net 2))
 (segment (start 197.173547 129.511092) (end 197.54509 129.882635) (width 0.25) (layer "B.Cu") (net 2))
 (segment (start 194.31 131.854061) (end 196.652969 129.511092) (width 0.25) (layer "B.Cu") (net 2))
 (segment (start 194.34 135.225) (end 194.31 135.255) (width 0.25) (layer "B.Cu") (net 2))
 (segment (start 221.625756 100.954244) (end 221.599214 100.980786) (width 0.25) (layer "B.Cu") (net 2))
 (segment (start 215.324961 100.965) (end 213.36 100.965) (width 0.25) (layer "B.Cu") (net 2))
 (segment (start 221.625756 93.597409) (end 221.625756 100.954244) (width 0.25) (layer "B.Cu") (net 2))
 (segment (start 212.645 96.52) (end 213.28 97.155) (width 0.25) (layer "B.Cu") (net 2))
 (segment (start 219.71 142.24) (end 219.71 129.54) (width 0.25) (layer "B.Cu") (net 2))
 (segment (start 217.645 128.27) (end 217.645 123.19) (width 0.25) (layer "B.Cu") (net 2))
 (segment (start 219.71 144.145) (end 219.71 142.24) (width 0.25) (layer "B.Cu") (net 2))
 (segment (start 218.44 140.97) (end 217.645 140.97) (width 0.25) (layer "B.Cu") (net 2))
 (segment (start 223.851007 103.836007) (end 223.52 103.505) (width 0.25) (layer "B.Cu") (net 2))
 (segment (start 212.09 144.225) (end 200.105 144.225) (width 0.25) (layer "B.Cu") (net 2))
 (segment (start 196.652969 129.511092) (end 197.173547 129.511092) (width 0.25) (layer "B.Cu") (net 2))
 (segment (start 221.583428 100.965) (end 222.25 101.631572) (width 0.25) (layer "B.Cu") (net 2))
 (segment (start 221.583428 100.965) (end 221.599214 100.980786) (width 0.25) (layer "B.Cu") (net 2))
 (segment (start 219.71 129.54) (end 218.44 128.27) (width 0.25) (layer "B.Cu") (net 2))
 (segment (start 219.71 142.24) (end 218.44 140.97) (width 0.25) (layer "B.Cu") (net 2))
 (segment (start 217.645 138.43) (end 216.535 138.43) (width 0.25) (layer "F.Cu") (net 7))
 (segment (start 207.645 147.32) (end 207.645 149.801218) (width 0.25) (layer "F.Cu") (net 7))
 (segment (start 207.645 149.801218) (end 208.28959 150.445808) (width 0.25) (layer "F.Cu") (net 7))
 (segment (start 216.535 138.43) (end 207.645 147.32) (width 0.25) (layer "F.Cu") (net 7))
 (segment (start 219.71 140.97) (end 210.185 150.495) (width 0.25) (layer "F.Cu") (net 8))
 (segment (start 225.585 133.35) (end 224.4725 133.35) (width 0.25) (layer "F.Cu") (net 8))
 (segment (start 224.4725 133.35) (end 219.71 138.1125) (width 0.25) (layer "F.Cu") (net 8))
 (segment (start 219.71 138.1125) (end 219.71 140.97) (width 0.25) (layer "F.Cu") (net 8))
 (segment (start 224.155 135.89) (end 220.345 139.7) (width 0.25) (layer "F.Cu") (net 9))
 (segment (start 220.345 142.24) (end 213.376952 149.208048) (width 0.25) (layer "F.Cu") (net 9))
 (segment (start 213.376952 149.208048) (end 213.376952 150.441902) (width 0.25) (layer "F.Cu") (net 9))
 (segment (start 220.345 139.7) (end 220.345 142.24) (width 0.25) (layer "F.Cu") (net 9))
 (segment (start 225.585 135.89) (end 224.155 135.89) (width 0.25) (layer "F.Cu") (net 9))
 (segment (start 215.92609 149.19891) (end 215.92609 150.445808) (width 0.25) (layer "F.Cu") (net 10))
 (segment (start 225.585 138.43) (end 224.155 138.43) (width 0.25) (layer "F.Cu") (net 10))
 (segment (start 224.155 138.43) (end 220.98 141.605) (width 0.25) (layer "F.Cu") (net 10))
 (segment (start 220.98 144.145) (end 215.92609 149.19891) (width 0.25) (layer "F.Cu") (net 10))
 (segment (start 220.98 141.605) (end 220.98 144.145) (width 0.25) (layer "F.Cu") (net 10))
 (segment (start 221.615 146.05) (end 221.615 142.875) (width 0.25) (layer "F.Cu") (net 11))
 (segment (start 221.615 142.875) (end 223.52 140.97) (width 0.25) (layer "F.Cu") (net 11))
 (segment (start 223.52 140.97) (end 225.585 140.97) (width 0.25) (layer "F.Cu") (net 11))
 (segment (start 218.47159 150.445808) (end 218.47159 149.19341) (width 0.25) (layer "F.Cu") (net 11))
 (segment (start 218.47159 149.19341) (end 221.615 146.05) (width 0.25) (layer "F.Cu") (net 11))
 (segment (start 209.55 132.08) (end 213.36 135.89) (width 0.25) (layer "F.Cu") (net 12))
 (segment (start 209.55 116.84) (end 209.55 132.08) (width 0.25) (layer "F.Cu") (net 12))
 (segment (start 213.36 135.89) (end 217.645 135.89) (width 0.25) (layer "F.Cu") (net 12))
 (via (at 209.55 116.84) (size 0.8) (drill 0.4) (layers "F.Cu" "B.Cu") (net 12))
 (segment (start 209.55 116.84) (end 202.565 116.84) (width 0.25) (layer "B.Cu") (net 12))
 (segment (start 202.565 116.84) (end 200.48602 114.76102) (width 0.25) (layer "B.Cu") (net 12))
 (segment (start 200.48602 114.76102) (end 200.48602 110.335004) (width 0.25) (layer "B.Cu") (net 12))
 (segment (start 217.645 133.35) (end 212.09 133.35) (width 0.25) (layer "F.Cu") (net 16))
 (segment (start 212.09 133.35) (end 210.82 132.08) (width 0.25) (layer "F.Cu") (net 16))
 (segment (start 210.82 132.08) (end 210.82 113.201089) (width 0.25) (layer "F.Cu") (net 16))
 (segment (start 210.82 113.201089) (end 207.954436 110.335525) (width 0.25) (layer "F.Cu") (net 16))
 (segment (start 216.535 130.81) (end 217.645 130.81) (width 0.25) (layer "F.Cu") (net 15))
 (segment (start 215.265 129.54) (end 216.535 130.81) (width 0.25) (layer "F.Cu") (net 15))
 (segment (start 215.265 110.49) (end 215.265 129.54) (width 0.25) (layer "F.Cu") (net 15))
 (via (at 215.265 110.49) (size 0.8) (drill 0.4) (layers "F.Cu" "B.Cu") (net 15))
 (segment (start 215.265 110.49) (end 215.355443 110.580443) (width 0.25) (layer "B.Cu") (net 15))
 (segment (start 215.355443 110.580443) (end 219.71 110.580443) (width 0.25) (layer "B.Cu") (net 15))
 (segment (start 219.71 110.580443) (end 219.954436 110.336007) (width 0.25) (layer "B.Cu") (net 15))
 (segment (start 205.74 142.24) (end 205.74 82.55) (width 0.25) (layer "F.Cu") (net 6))
 (segment (start 204.086891 80.896891) (end 198.765756 80.896891) (width 0.25) (layer "F.Cu") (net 6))
 (segment (start 202.565 150.495) (end 202.565 145.415) (width 0.25) (layer "F.Cu") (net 6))
 (segment (start 205.74 82.55) (end 204.086891 80.896891) (width 0.25) (layer "F.Cu") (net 6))
 (segment (start 202.565 145.415) (end 205.74 142.24) (width 0.25) (layer "F.Cu") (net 6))
 (segment (start 198.765756 96.530756) (end 198.755 96.52) (width 0.25) (layer "F.Cu") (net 14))
 (segment (start 198.765756 93.596891) (end 198.755 96.52) (width 0.25) (layer "F.Cu") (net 14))
 (segment (start 202.565 101.6) (end 198.765756 97.800756) (width 0.25) (layer "F.Cu") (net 14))
 (segment (start 198.765756 97.800756) (end 198.765756 96.530756) (width 0.25) (layer "F.Cu") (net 14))
 (segment (start 199.39 121.285) (end 199.39 116.205) (width 0.25) (layer "F.Cu") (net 14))
 (segment (start 202.565 113.03) (end 202.565 101.6) (width 0.25) (layer "F.Cu") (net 14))
 (segment (start 199.39 116.205) (end 202.565 113.03) (width 0.25) (layer "F.Cu") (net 14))
 (via (at 199.39 121.285) (size 0.6) (drill 0.3) (layers "F.Cu" "B.Cu") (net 14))
 (via (at 198.755 96.52) (size 0.6) (drill 0.3) (layers "F.Cu" "B.Cu") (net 14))
 (segment (start 223.52 123.19) (end 225.585 123.19) (width 0.25) (layer "B.Cu") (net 14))
 (segment (start 199.39 121.285) (end 221.615 121.285) (width 0.25) (layer "B.Cu") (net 14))
 (segment (start 221.615 121.285) (end 223.52 123.19) (width 0.25) (layer "B.Cu") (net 14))
 (segment (start 199.39 121.285) (end 199.39 130.078) (width 0.25) (layer "B.Cu") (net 14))
 (segment (start 207.645 96.52) (end 198.755 96.52) (width 0.25) (layer "B.Cu") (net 14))
 (segment (start 199.39 130.078) (end 199.457 130.145) (width 0.25) (layer "B.Cu") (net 14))
 (segment (start 203.835 52.07) (end 210.185 52.07) (width 0.25) (layer "F.Cu") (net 13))
 (segment (start 210.185 52.07) (end 211.383066 50.871934) (width 0.25) (layer "F.Cu") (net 13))
 (segment (start 211.383066 50.871934) (end 211.383066 45.453472) (width 0.25) (layer "F.Cu") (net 13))
 (segment (start 199.815756 68.196891) (end 201.295 66.717647) (width 0.25) (layer "F.Cu") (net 13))
 (segment (start 198.765756 68.196891) (end 199.815756 68.196891) (width 0.25) (layer "F.Cu") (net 13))
 (segment (start 201.295 66.717647) (end 201.295 52.07) (width 0.25) (layer "F.Cu") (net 13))
 (segment (start 200.66 137.795) (end 203.2 137.795) (width 0.25) (layer "F.Cu") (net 3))
 (segment (start 199.457 136.592) (end 200.66 137.795) (width 0.25) (layer "F.Cu") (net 3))
 (segment (start 204.47 136.525) (end 204.47 86.995) (width 0.25) (layer "F.Cu") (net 3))
 (segment (start 203.2 85.725) (end 199.439947 85.725) (width 0.25) (layer "F.Cu") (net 3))
 (segment (start 199.457 135.225) (end 199.457 136.592) (width 0.25) (layer "F.Cu") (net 3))
 (segment (start 204.47 86.995) (end 203.2 85.725) (width 0.25) (layer "F.Cu") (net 3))
 (segment (start 203.2 137.795) (end 204.47 136.525) (width 0.25) (layer "F.Cu") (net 3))
 (segment (start 199.439947 85.725) (end 199.363599 85.801348) (width 0.25) (layer "F.Cu") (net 3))
 (segment (start 199.43988 88.265) (end 199.363505 88.341375) (width 0.25) (layer "F.Cu") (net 4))
 (segment (start 201.997 135.225) (end 203.835 133.387) (width 0.25) (layer "F.Cu") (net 4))
 (segment (start 203.835 89.535) (end 202.565 88.265) (width 0.25) (layer "F.Cu") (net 4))
 (segment (start 203.835 133.387) (end 203.835 89.535) (width 0.25) (layer "F.Cu") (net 4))
 (segment (start 202.565 88.265) (end 199.43988 88.265) (width 0.25) (layer "F.Cu") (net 4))
 (segment (start 203.241891 92.116891) (end 203.241891 93.772932) (width 0.25) (layer "F.Cu") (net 20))
 (segment (start 203.2 128.942) (end 201.997 130.145) (width 0.25) (layer "F.Cu") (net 20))
 (segment (start 203.2 93.814823) (end 203.2 128.942) (width 0.25) (layer "F.Cu") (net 20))
 (segment (start 198.765756 91.056891) (end 202.181891 91.056891) (width 0.25) (layer "F.Cu") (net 20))
 (segment (start 202.181891 91.056891) (end 203.241891 92.116891) (width 0.25) (layer "F.Cu") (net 20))
 (segment (start 203.241891 93.772932) (end 203.2 93.814823) (width 0.25) (layer "F.Cu") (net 20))
 (segment (start 202.565 53.34) (end 203.835 54.61) (width 0.25) (layer "F.Cu") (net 1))
 (segment (start 201.043109 75.816891) (end 198.765756 75.816891) (width 0.25) (layer "F.Cu") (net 1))
 (segment (start 203.835 54.61) (end 203.835 57.15) (width 0.25) (layer "F.Cu") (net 1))
 (segment (start 203.835 73.025) (end 201.043109 75.816891) (width 0.25) (layer "F.Cu") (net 1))
 (segment (start 203.835 62.23) (end 203.835 73.025) (width 0.25) (layer "F.Cu") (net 1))
 (segment (start 219.457591 83.437409) (end 221.625756 83.437409) (width 0.25) (layer "F.Cu") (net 18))
 (segment (start 217.805 113.665) (end 217.805 85.09) (width 0.25) (layer "F.Cu") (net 18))
 (segment (start 225.585 125.73) (end 222.25 125.73) (width 0.25) (layer "F.Cu") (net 18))
 (segment (start 222.25 125.73) (end 220.98 124.46) (width 0.25) (layer "F.Cu") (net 18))
 (segment (start 217.805 85.09) (end 219.457591 83.437409) (width 0.25) (layer "F.Cu") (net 18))
 (segment (start 220.98 124.46) (end 220.98 116.84) (width 0.25) (layer "F.Cu") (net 18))
 (segment (start 220.98 116.84) (end 217.805 113.665) (width 0.25) (layer "F.Cu") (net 18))
 (segment (start 216.535 115.57) (end 216.535 84.455) (width 0.25) (layer "F.Cu") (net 17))
 (segment (start 225.585 128.27) (end 224.95 128.905) (width 0.25) (layer "F.Cu") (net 17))
 (segment (start 220.092591 80.897409) (end 221.625756 80.897409) (width 0.25) (layer "F.Cu") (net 17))
 (segment (start 219.075 126.365) (end 219.075 118.11) (width 0.25) (layer "F.Cu") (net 17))
 (segment (start 221.615 128.905) (end 219.075 126.365) (width 0.25) (layer "F.Cu") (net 17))
 (segment (start 224.95 128.905) (end 221.615 128.905) (width 0.25) (layer "F.Cu") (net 17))
 (segment (start 216.535 84.455) (end 220.092591 80.897409) (width 0.25) (layer "F.Cu") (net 17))
 (segment (start 219.075 118.11) (end 216.535 115.57) (width 0.25) (layer "F.Cu") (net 17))
 (segment (start 204.101528 45.453472) (end 208.843066 45.453472) (width 0.25) (layer "F.Cu") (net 19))
 (segment (start 198.755 50.8) (end 204.101528 45.453472) (width 0.25) (layer "F.Cu") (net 19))
 (segment (start 198.755 57.15) (end 198.755 50.8) (width 0.25) (layer "F.Cu") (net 19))
 (segment (start 198.765756 62.240756) (end 198.755 62.23) (width 0.25) (layer "F.Cu") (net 19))
 (segment (start 198.765756 65.656891) (end 198.765756 62.240756) (width 0.25) (layer "F.Cu") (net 19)))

